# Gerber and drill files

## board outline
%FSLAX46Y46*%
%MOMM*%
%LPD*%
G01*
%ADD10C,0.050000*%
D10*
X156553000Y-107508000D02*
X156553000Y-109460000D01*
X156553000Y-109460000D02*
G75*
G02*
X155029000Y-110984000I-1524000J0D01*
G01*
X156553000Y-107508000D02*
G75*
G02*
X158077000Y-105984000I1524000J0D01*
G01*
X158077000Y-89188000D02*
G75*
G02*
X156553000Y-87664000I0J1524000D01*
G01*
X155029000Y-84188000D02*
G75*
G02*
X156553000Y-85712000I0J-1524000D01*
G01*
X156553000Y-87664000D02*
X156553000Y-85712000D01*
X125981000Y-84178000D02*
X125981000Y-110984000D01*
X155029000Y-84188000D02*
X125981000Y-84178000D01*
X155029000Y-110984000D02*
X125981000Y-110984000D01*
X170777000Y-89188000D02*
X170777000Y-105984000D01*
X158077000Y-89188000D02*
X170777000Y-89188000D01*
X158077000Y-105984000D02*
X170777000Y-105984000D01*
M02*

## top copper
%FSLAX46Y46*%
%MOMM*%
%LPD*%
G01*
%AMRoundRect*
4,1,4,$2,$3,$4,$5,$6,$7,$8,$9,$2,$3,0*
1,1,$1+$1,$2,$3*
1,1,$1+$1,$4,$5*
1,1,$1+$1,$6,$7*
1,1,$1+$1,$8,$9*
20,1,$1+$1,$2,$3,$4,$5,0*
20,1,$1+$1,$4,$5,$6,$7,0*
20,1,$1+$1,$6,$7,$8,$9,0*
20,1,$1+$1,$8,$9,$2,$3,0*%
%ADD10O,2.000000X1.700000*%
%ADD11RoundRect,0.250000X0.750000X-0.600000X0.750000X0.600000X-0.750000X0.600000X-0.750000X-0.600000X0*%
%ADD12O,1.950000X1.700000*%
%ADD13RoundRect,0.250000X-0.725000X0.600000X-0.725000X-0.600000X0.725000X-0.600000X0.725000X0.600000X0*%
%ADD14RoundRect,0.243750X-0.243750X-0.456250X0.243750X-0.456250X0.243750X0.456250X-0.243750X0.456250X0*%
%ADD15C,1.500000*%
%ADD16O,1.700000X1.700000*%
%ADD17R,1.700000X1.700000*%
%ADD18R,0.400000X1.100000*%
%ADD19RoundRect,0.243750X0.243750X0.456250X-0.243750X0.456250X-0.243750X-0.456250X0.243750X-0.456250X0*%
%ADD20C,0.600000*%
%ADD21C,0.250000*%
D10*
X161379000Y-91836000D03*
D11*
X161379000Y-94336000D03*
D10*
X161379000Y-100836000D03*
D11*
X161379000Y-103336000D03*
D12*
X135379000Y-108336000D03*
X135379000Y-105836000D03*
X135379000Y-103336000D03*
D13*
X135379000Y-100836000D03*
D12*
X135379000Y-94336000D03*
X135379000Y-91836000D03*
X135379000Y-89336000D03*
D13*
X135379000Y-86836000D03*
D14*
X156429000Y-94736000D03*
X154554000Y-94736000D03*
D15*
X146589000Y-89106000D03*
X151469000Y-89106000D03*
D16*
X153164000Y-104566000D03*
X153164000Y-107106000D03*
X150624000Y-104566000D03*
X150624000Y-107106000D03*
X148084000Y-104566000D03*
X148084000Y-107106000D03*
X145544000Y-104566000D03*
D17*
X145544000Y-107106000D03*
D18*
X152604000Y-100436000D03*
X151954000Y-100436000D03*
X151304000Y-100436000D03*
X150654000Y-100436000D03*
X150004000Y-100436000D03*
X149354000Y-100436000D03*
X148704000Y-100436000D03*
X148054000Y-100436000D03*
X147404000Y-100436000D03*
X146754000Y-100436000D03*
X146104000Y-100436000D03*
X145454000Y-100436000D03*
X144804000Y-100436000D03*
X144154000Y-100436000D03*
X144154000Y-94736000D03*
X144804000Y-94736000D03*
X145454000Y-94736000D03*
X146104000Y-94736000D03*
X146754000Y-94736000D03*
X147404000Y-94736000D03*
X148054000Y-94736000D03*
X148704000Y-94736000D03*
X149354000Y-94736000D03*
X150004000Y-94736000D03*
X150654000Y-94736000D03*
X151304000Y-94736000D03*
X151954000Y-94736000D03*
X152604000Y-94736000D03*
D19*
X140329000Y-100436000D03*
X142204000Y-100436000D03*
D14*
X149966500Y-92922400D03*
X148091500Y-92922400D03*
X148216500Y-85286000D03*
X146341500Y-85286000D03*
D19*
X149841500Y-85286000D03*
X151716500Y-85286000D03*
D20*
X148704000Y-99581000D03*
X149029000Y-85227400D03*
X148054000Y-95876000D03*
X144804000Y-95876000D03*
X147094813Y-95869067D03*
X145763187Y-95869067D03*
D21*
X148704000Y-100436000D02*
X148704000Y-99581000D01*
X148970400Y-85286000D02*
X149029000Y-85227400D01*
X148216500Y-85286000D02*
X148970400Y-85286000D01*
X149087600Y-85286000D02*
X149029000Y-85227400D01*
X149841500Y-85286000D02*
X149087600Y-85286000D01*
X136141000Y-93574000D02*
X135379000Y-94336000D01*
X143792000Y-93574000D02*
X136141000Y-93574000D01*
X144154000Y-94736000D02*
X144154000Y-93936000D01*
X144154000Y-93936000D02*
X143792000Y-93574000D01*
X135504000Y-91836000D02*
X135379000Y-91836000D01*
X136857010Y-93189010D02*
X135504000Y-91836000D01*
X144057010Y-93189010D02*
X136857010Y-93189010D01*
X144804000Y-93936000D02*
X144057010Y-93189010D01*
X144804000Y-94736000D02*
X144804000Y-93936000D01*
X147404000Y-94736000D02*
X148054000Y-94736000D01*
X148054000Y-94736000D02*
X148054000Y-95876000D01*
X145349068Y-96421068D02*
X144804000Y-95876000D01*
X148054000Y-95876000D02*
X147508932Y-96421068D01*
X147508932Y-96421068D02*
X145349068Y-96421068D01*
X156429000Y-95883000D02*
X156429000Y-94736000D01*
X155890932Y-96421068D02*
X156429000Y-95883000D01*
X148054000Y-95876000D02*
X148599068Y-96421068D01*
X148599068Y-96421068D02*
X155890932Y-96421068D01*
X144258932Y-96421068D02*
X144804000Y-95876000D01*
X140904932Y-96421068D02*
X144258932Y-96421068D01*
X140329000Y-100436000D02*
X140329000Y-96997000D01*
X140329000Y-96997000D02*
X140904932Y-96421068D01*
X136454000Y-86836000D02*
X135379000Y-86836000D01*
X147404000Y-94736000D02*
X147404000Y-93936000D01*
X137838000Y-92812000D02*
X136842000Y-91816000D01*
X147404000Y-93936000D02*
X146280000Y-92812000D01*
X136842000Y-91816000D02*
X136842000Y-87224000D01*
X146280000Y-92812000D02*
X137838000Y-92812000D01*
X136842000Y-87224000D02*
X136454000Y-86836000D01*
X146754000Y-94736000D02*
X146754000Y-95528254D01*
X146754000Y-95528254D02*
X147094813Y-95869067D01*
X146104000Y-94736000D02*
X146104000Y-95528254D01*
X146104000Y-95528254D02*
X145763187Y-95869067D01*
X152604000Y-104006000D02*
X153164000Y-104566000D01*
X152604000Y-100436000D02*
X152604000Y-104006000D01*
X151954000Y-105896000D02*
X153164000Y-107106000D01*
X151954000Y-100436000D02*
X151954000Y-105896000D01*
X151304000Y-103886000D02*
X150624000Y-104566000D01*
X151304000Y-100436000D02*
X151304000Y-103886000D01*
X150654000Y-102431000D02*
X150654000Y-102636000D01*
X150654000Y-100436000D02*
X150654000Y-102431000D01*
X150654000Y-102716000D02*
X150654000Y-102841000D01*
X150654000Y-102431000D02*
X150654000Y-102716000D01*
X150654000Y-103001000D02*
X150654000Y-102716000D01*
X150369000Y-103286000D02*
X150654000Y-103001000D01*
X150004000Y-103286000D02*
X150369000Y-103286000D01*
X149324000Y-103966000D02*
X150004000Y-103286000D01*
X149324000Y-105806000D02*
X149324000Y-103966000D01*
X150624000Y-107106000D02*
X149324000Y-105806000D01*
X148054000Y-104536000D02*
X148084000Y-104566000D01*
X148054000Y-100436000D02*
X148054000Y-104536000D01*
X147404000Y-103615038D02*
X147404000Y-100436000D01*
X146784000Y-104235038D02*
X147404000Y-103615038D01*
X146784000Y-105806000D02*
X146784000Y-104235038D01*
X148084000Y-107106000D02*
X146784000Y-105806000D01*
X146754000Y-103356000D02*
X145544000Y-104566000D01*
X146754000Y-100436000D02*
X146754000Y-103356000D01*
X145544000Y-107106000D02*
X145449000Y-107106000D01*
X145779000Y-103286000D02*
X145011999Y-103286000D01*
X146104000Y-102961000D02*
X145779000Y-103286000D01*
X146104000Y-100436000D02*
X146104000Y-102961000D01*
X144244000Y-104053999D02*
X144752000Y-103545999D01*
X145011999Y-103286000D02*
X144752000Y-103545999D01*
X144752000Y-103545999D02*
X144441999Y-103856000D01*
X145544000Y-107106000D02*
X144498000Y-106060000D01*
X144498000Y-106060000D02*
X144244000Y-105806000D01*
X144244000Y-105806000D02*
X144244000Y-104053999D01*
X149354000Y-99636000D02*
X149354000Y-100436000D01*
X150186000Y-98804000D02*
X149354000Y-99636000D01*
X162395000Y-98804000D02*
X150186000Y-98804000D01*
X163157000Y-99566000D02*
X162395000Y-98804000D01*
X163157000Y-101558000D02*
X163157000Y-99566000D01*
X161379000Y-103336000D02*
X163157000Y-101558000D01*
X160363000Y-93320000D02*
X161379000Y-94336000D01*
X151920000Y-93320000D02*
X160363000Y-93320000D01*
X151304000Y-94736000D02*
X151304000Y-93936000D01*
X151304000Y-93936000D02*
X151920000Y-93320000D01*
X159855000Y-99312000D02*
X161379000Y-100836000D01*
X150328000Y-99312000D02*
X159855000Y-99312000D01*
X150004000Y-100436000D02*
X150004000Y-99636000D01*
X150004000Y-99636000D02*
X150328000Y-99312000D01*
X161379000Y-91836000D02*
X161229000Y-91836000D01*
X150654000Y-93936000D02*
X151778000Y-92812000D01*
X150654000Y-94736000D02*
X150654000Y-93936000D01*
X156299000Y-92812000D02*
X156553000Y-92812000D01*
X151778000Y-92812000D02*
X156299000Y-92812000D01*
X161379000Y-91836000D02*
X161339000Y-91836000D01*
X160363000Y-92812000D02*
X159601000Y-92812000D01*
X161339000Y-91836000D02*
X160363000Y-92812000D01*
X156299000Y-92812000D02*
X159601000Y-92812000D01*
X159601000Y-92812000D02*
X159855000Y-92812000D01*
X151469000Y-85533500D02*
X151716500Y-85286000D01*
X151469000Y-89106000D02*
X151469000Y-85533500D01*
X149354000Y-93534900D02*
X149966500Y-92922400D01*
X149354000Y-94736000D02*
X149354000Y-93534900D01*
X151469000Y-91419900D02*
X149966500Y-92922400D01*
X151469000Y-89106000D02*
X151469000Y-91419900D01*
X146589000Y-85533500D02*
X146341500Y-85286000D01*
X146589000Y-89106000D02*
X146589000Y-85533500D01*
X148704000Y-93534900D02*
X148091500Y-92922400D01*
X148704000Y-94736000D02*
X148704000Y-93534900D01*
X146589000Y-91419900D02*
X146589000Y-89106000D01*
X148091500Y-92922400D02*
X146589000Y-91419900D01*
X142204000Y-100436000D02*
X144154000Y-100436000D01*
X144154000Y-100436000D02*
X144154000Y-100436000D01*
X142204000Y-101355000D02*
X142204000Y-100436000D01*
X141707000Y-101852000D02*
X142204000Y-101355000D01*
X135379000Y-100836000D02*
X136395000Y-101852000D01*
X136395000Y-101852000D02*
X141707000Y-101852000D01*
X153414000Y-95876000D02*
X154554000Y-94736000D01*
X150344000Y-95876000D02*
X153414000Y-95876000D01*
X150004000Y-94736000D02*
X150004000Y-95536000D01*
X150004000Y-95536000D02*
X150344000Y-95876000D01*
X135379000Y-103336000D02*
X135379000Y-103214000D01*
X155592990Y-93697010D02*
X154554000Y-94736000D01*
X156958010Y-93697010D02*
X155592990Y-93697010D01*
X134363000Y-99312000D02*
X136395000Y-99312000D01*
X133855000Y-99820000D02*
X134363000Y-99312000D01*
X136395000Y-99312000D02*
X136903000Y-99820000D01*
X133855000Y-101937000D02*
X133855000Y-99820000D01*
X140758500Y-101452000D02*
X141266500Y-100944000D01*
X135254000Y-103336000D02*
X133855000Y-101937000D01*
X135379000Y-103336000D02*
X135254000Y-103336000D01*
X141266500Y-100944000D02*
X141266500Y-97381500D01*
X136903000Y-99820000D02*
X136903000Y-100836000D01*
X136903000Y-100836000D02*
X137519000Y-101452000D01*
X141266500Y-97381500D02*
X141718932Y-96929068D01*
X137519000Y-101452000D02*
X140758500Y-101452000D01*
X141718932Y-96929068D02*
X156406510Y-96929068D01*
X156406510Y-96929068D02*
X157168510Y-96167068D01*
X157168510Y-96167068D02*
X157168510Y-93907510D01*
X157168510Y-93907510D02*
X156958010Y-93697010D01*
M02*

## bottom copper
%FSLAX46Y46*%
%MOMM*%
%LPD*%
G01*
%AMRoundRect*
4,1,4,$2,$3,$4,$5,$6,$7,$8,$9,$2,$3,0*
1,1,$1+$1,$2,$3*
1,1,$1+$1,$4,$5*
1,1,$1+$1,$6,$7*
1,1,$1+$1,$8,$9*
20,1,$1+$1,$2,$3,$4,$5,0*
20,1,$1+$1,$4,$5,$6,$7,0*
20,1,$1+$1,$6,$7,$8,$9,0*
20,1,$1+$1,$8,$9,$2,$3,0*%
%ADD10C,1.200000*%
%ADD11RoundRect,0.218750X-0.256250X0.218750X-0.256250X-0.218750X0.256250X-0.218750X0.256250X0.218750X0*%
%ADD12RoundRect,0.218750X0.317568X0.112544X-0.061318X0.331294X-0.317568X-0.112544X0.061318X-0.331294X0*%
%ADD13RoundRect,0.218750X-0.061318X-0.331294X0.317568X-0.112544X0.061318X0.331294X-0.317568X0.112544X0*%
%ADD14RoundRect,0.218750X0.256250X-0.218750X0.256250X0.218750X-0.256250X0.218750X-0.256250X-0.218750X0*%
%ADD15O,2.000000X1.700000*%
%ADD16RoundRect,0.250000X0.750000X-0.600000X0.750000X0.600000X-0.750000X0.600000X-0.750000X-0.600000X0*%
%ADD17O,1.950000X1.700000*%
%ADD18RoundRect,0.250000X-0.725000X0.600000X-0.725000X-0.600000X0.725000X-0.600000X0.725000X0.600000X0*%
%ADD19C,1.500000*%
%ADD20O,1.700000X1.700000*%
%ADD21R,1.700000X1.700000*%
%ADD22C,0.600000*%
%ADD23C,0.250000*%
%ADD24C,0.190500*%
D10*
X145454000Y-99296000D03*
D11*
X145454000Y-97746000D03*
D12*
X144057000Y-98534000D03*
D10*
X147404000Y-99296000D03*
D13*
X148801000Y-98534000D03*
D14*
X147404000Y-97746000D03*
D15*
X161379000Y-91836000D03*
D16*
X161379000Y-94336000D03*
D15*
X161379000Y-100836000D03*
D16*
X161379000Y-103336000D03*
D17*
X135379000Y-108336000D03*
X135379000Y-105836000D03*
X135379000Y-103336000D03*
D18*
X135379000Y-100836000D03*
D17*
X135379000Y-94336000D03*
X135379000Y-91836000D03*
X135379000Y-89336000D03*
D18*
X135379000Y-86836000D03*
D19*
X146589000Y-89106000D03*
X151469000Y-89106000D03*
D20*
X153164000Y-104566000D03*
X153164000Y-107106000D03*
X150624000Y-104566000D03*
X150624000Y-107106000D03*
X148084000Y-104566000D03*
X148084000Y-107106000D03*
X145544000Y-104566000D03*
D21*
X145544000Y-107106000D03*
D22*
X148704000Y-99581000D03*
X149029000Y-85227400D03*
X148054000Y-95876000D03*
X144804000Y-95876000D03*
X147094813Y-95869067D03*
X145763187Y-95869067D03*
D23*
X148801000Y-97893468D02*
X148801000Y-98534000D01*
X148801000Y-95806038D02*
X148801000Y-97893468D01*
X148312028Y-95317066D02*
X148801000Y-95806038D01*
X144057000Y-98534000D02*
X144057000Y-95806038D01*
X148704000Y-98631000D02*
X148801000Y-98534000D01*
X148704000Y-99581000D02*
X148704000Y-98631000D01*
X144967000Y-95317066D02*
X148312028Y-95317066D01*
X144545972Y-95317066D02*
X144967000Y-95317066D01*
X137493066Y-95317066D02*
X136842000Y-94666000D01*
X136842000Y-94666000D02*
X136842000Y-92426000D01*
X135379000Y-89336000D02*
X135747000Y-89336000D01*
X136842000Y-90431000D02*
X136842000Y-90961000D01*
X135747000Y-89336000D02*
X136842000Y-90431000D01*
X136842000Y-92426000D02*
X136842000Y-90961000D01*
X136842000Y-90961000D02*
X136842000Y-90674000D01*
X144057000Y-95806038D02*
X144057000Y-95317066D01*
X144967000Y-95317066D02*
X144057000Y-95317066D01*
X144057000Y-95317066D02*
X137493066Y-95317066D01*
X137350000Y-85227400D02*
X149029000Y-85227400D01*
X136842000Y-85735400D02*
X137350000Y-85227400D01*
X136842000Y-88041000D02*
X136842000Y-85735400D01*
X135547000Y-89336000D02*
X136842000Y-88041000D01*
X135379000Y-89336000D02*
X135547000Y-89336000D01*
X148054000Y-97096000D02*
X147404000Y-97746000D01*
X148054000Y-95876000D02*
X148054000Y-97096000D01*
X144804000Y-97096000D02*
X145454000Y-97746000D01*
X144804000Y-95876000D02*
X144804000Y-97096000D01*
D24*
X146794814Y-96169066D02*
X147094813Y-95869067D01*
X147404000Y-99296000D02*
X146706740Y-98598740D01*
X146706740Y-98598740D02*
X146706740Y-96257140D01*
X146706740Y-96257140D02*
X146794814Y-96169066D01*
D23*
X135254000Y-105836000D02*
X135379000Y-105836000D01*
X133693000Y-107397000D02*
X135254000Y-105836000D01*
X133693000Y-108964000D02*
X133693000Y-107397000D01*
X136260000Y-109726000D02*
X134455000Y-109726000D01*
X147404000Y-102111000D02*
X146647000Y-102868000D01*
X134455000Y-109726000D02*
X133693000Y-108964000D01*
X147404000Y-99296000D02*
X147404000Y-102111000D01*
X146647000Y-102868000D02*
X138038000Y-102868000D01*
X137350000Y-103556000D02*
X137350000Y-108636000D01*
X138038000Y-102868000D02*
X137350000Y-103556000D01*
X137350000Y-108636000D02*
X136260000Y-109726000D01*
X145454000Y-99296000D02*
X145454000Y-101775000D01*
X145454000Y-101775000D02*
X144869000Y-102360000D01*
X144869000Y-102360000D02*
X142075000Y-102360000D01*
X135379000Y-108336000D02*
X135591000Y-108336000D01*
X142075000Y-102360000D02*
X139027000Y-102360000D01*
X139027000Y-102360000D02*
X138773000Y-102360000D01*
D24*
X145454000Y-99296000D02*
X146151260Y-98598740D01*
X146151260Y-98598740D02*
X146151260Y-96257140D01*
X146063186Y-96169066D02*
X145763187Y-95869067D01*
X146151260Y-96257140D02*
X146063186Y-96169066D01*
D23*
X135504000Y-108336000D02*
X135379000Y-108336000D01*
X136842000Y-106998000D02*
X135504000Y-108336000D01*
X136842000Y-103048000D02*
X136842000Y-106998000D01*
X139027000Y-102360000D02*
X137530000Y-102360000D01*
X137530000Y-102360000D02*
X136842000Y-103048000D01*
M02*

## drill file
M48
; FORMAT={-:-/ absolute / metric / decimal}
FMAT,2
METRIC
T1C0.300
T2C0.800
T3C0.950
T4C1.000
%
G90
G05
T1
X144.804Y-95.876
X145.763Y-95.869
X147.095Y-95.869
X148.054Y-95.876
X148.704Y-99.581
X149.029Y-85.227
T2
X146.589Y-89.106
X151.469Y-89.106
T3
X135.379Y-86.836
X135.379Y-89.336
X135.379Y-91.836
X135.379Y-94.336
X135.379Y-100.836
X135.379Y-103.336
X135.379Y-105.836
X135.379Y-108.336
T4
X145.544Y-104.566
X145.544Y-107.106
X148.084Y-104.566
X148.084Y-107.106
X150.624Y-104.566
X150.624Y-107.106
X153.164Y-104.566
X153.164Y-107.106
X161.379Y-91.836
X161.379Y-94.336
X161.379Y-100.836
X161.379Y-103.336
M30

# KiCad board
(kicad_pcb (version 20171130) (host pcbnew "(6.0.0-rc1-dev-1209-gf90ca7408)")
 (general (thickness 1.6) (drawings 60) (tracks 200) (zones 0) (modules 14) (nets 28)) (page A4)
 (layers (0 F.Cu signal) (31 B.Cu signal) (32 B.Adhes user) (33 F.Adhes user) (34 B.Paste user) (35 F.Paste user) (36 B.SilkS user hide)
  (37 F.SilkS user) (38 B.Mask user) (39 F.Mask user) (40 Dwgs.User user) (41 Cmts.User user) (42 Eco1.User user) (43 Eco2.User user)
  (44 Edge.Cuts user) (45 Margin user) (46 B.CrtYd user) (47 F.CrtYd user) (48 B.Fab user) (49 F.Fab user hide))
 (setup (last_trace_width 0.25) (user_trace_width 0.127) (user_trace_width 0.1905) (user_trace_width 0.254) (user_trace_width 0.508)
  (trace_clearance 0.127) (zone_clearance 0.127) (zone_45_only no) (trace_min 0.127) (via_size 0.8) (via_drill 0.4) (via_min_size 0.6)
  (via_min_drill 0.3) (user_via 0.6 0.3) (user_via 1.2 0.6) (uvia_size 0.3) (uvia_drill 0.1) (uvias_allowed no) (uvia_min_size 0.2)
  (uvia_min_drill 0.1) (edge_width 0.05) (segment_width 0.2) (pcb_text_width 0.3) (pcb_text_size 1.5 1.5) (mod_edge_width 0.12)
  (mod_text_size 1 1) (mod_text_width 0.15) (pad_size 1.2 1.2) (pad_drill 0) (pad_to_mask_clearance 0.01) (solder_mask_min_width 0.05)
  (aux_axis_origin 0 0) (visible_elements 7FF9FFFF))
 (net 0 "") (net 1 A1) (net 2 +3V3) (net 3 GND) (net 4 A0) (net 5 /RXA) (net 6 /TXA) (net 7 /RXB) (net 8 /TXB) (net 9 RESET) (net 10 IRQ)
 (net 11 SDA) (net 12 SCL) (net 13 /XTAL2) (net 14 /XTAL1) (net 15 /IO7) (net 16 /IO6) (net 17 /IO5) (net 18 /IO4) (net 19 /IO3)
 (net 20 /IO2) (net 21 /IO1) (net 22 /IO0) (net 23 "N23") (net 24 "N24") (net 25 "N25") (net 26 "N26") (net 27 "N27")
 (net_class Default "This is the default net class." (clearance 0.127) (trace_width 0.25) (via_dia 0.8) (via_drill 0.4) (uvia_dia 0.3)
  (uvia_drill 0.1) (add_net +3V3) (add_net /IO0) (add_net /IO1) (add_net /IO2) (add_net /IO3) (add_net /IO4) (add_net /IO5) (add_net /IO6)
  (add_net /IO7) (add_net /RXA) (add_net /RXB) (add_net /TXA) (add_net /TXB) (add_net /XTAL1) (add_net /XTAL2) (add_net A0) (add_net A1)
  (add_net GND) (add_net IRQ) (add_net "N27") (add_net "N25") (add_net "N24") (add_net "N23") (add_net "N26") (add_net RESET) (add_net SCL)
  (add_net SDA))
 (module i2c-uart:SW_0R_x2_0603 (layer B.Cu) (at 145.454 99.296)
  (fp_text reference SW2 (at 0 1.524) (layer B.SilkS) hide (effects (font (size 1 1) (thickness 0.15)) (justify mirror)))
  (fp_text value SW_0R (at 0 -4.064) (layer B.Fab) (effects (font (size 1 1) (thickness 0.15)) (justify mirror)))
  (pad 2 smd circle (at 0 0) (size 1.2 1.2) (layers B.Cu B.Paste B.Mask) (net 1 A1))
  (pad 1 smd roundrect (at 0 -1.55 270) (size 0.875 0.95) (layers B.Cu B.Paste B.Mask) (roundrect_rratio 0.25) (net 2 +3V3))
  (pad 3 smd roundrect (at -1.397 -0.762 150) (size 0.875 0.95) (layers B.Cu B.Paste B.Mask) (roundrect_rratio 0.25) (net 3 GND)))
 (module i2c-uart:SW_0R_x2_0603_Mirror (layer B.Cu) (at 147.404 99.296 180)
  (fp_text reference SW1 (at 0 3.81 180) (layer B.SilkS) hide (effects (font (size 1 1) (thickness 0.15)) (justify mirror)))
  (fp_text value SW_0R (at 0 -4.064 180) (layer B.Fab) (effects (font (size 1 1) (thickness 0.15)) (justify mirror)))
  (pad 2 smd circle (at 0 0 180) (size 1.2 1.2) (layers B.Cu B.Paste B.Mask) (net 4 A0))
  (pad 3 smd roundrect (at -1.397 0.762 30) (size 0.875 0.95) (layers B.Cu B.Paste B.Mask) (roundrect_rratio 0.25) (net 3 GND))
  (pad 1 smd roundrect (at 0 1.55 90) (size 0.875 0.95) (layers B.Cu B.Paste B.Mask) (roundrect_rratio 0.25) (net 2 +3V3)))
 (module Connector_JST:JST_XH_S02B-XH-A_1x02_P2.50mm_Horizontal (layer F.Cu) (at 161.379 94.336 90)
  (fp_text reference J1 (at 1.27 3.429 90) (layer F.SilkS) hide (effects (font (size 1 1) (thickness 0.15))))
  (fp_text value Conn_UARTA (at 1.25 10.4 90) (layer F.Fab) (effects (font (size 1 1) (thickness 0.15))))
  (pad 2 thru_hole oval (at 2.5 0 90) (size 1.7 2) (drill 1) (layers *.Cu *.Mask) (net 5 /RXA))
  (pad 1 thru_hole roundrect (at 0 0 90) (size 1.7 2) (drill 1) (layers *.Cu *.Mask) (roundrect_rratio 0.147059) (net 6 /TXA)))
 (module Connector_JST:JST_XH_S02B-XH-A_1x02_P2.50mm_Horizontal (layer F.Cu) (at 161.379 103.336 90)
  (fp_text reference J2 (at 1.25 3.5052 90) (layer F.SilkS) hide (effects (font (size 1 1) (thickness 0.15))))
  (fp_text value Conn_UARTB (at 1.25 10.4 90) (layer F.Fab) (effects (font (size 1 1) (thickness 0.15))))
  (pad 2 thru_hole oval (at 2.5 0 90) (size 1.7 2) (drill 1) (layers *.Cu *.Mask) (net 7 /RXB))
  (pad 1 thru_hole roundrect (at 0 0 90) (size 1.7 2) (drill 1) (layers *.Cu *.Mask) (roundrect_rratio 0.147059) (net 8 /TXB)))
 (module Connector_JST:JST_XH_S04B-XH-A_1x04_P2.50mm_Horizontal (layer F.Cu) (at 135.379 100.836 270)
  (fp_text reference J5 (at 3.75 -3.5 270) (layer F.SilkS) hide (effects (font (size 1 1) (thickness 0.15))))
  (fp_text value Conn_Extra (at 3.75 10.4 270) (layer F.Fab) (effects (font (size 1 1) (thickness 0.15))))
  (pad 4 thru_hole oval (at 7.5 0 270) (size 1.7 1.95) (drill 0.95) (layers *.Cu *.Mask) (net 1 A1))
  (pad 3 thru_hole oval (at 5 0 270) (size 1.7 1.95) (drill 0.95) (layers *.Cu *.Mask) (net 4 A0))
  (pad 2 thru_hole oval (at 2.5 0 270) (size 1.7 1.95) (drill 0.95) (layers *.Cu *.Mask) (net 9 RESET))
  (pad 1 thru_hole roundrect (at 0 0 270) (size 1.7 1.95) (drill 0.95) (layers *.Cu *.Mask) (roundrect_rratio 0.147059) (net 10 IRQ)))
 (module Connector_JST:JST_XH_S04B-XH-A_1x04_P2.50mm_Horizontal (layer F.Cu) (at 135.379 86.836 270)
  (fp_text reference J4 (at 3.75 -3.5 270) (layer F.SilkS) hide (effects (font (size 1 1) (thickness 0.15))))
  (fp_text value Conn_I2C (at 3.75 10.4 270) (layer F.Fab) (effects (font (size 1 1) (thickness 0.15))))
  (pad 4 thru_hole oval (at 7.5 0 270) (size 1.7 1.95) (drill 0.95) (layers *.Cu *.Mask) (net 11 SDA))
  (pad 3 thru_hole oval (at 5 0 270) (size 1.7 1.95) (drill 0.95) (layers *.Cu *.Mask) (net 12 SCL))
  (pad 2 thru_hole oval (at 2.5 0 270) (size 1.7 1.95) (drill 0.95) (layers *.Cu *.Mask) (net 3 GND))
  (pad 1 thru_hole roundrect (at 0 0 270) (size 1.7 1.95) (drill 0.95) (layers *.Cu *.Mask) (roundrect_rratio 0.147059) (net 2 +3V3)))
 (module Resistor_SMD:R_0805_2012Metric (layer F.Cu) (at 155.4915 94.736)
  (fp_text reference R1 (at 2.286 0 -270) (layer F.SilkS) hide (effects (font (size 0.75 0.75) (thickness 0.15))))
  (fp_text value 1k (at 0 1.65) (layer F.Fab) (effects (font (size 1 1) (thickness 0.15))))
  (pad 2 smd roundrect (at 0.9375 0) (size 0.975 1.4) (layers F.Cu F.Paste F.Mask) (roundrect_rratio 0.25) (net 2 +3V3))
  (pad 1 smd roundrect (at -0.9375 0) (size 0.975 1.4) (layers F.Cu F.Paste F.Mask) (roundrect_rratio 0.25) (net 9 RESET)))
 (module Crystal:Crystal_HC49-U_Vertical (layer F.Cu) (at 151.469 89.106 180)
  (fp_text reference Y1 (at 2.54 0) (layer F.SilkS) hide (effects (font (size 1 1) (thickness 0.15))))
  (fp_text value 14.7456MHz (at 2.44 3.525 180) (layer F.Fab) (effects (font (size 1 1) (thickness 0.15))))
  (pad 2 thru_hole circle (at 4.88 0 180) (size 1.5 1.5) (drill 0.8) (layers *.Cu *.Mask) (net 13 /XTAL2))
  (pad 1 thru_hole circle (at 0 0 180) (size 1.5 1.5) (drill 0.8) (layers *.Cu *.Mask) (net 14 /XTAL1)))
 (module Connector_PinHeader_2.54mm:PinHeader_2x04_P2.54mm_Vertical (layer F.Cu) (at 145.544 107.106 90)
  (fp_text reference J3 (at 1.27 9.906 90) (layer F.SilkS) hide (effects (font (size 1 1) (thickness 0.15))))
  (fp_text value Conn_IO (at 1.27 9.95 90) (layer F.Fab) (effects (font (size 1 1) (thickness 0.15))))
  (pad 8 thru_hole oval (at 2.54 7.62 90) (size 1.7 1.7) (drill 1) (layers *.Cu *.Mask) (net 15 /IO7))
  (pad 7 thru_hole oval (at 0 7.62 90) (size 1.7 1.7) (drill 1) (layers *.Cu *.Mask) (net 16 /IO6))
  (pad 6 thru_hole oval (at 2.54 5.08 90) (size 1.7 1.7) (drill 1) (layers *.Cu *.Mask) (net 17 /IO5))
  (pad 5 thru_hole oval (at 0 5.08 90) (size 1.7 1.7) (drill 1) (layers *.Cu *.Mask) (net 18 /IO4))
  (pad 4 thru_hole oval (at 2.54 2.54 90) (size 1.7 1.7) (drill 1) (layers *.Cu *.Mask) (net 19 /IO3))
  (pad 3 thru_hole oval (at 0 2.54 90) (size 1.7 1.7) (drill 1) (layers *.Cu *.Mask) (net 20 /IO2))
  (pad 2 thru_hole oval (at 2.54 0 90) (size 1.7 1.7) (drill 1) (layers *.Cu *.Mask) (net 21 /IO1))
  (pad 1 thru_hole rect (at 0 0 90) (size 1.7 1.7) (drill 1) (layers *.Cu *.Mask) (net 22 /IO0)))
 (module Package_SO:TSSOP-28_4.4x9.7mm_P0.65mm (layer F.Cu) (at 148.379 97.586 270)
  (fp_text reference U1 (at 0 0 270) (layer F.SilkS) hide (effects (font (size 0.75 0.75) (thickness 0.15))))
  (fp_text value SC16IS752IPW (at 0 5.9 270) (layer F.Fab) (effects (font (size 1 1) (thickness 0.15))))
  (pad 28 smd rect (at 2.85 -4.225 270) (size 1.1 0.4) (layers F.Cu F.Paste F.Mask) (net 15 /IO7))
  (pad 27 smd rect (at 2.85 -3.575 270) (size 1.1 0.4) (layers F.Cu F.Paste F.Mask) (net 16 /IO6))
  (pad 26 smd rect (at 2.85 -2.925 270) (size 1.1 0.4) (layers F.Cu F.Paste F.Mask) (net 17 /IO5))
  (pad 25 smd rect (at 2.85 -2.275 270) (size 1.1 0.4) (layers F.Cu F.Paste F.Mask) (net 18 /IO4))
  (pad 24 smd rect (at 2.85 -1.625 270) (size 1.1 0.4) (layers F.Cu F.Paste F.Mask) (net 7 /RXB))
  (pad 23 smd rect (at 2.85 -0.975 270) (size 1.1 0.4) (layers F.Cu F.Paste F.Mask) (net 8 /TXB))
  (pad 22 smd rect (at 2.85 -0.325 270) (size 1.1 0.4) (layers F.Cu F.Paste F.Mask) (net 3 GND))
  (pad 21 smd rect (at 2.85 0.325 270) (size 1.1 0.4) (layers F.Cu F.Paste F.Mask) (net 19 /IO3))
  (pad 20 smd rect (at 2.85 0.975 270) (size 1.1 0.4) (layers F.Cu F.Paste F.Mask) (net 20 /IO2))
  (pad 19 smd rect (at 2.85 1.625 270) (size 1.1 0.4) (layers F.Cu F.Paste F.Mask) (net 21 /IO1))
  (pad 18 smd rect (at 2.85 2.275 270) (size 1.1 0.4) (layers F.Cu F.Paste F.Mask) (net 22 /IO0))
  (pad 17 smd rect (at 2.85 2.925 270) (size 1.1 0.4) (layers F.Cu F.Paste F.Mask) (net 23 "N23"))
  (pad 16 smd rect (at 2.85 3.575 270) (size 1.1 0.4) (layers F.Cu F.Paste F.Mask) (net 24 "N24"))
  (pad 15 smd rect (at 2.85 4.225 270) (size 1.1 0.4) (layers F.Cu F.Paste F.Mask) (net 10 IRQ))
  (pad 14 smd rect (at -2.85 4.225 270) (size 1.1 0.4) (layers F.Cu F.Paste F.Mask) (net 11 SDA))
  (pad 13 smd rect (at -2.85 3.575 270) (size 1.1 0.4) (layers F.Cu F.Paste F.Mask) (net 12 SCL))
  (pad 12 smd rect (at -2.85 2.925 270) (size 1.1 0.4) (layers F.Cu F.Paste F.Mask) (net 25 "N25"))
  (pad 11 smd rect (at -2.85 2.275 270) (size 1.1 0.4) (layers F.Cu F.Paste F.Mask) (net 1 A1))
  (pad 10 smd rect (at -2.85 1.625 270) (size 1.1 0.4) (layers F.Cu F.Paste F.Mask) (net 4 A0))
  (pad 9 smd rect (at -2.85 0.975 270) (size 1.1 0.4) (layers F.Cu F.Paste F.Mask) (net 2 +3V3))
  (pad 8 smd rect (at -2.85 0.325 270) (size 1.1 0.4) (layers F.Cu F.Paste F.Mask) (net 2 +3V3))
  (pad 7 smd rect (at -2.85 -0.325 270) (size 1.1 0.4) (layers F.Cu F.Paste F.Mask) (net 13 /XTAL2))
  (pad 6 smd rect (at -2.85 -0.975 270) (size 1.1 0.4) (layers F.Cu F.Paste F.Mask) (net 14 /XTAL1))
  (pad 5 smd rect (at -2.85 -1.625 270) (size 1.1 0.4) (layers F.Cu F.Paste F.Mask) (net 9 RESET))
  (pad 4 smd rect (at -2.85 -2.275 270) (size 1.1 0.4) (layers F.Cu F.Paste F.Mask) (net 5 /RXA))
  (pad 3 smd rect (at -2.85 -2.925 270) (size 1.1 0.4) (layers F.Cu F.Paste F.Mask) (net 6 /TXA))
  (pad 2 smd rect (at -2.85 -3.575 270) (size 1.1 0.4) (layers F.Cu F.Paste F.Mask) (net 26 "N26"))
  (pad 1 smd rect (at -2.85 -4.225 270) (size 1.1 0.4) (layers F.Cu F.Paste F.Mask) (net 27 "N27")))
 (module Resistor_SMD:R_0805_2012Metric (layer F.Cu) (at 141.2665 100.436 180)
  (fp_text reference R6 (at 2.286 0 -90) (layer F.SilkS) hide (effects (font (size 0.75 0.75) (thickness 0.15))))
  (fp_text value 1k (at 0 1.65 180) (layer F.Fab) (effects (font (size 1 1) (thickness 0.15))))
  (pad 2 smd roundrect (at 0.9375 0 180) (size 0.975 1.4) (layers F.Cu F.Paste F.Mask) (roundrect_rratio 0.25) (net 2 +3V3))
  (pad 1 smd roundrect (at -0.9375 0 180) (size 0.975 1.4) (layers F.Cu F.Paste F.Mask) (roundrect_rratio 0.25) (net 10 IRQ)))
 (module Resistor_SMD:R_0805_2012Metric (layer F.Cu) (at 149.029 92.9224)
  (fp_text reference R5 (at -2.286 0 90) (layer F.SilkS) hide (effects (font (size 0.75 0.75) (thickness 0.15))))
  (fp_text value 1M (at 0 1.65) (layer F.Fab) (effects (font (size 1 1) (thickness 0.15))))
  (pad 2 smd roundrect (at 0.9375 0) (size 0.975 1.4) (layers F.Cu F.Paste F.Mask) (roundrect_rratio 0.25) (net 14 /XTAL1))
  (pad 1 smd roundrect (at -0.9375 0) (size 0.975 1.4) (layers F.Cu F.Paste F.Mask) (roundrect_rratio 0.25) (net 13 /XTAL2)))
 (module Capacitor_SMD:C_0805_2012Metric (layer F.Cu) (at 147.279 85.286)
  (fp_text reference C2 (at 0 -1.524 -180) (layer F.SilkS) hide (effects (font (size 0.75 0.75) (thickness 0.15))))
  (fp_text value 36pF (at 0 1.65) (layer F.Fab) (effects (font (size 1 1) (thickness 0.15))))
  (pad 2 smd roundrect (at 0.9375 0) (size 0.975 1.4) (layers F.Cu F.Paste F.Mask) (roundrect_rratio 0.25) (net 3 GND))
  (pad 1 smd roundrect (at -0.9375 0) (size 0.975 1.4) (layers F.Cu F.Paste F.Mask) (roundrect_rratio 0.25) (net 13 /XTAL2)))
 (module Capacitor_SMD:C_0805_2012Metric (layer F.Cu) (at 150.779 85.286 180)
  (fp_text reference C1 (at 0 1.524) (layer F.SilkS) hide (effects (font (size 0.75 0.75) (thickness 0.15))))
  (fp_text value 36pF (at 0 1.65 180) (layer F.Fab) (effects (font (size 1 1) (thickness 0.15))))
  (pad 2 smd roundrect (at 0.9375 0 180) (size 0.975 1.4) (layers F.Cu F.Paste F.Mask) (roundrect_rratio 0.25) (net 3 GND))
  (pad 1 smd roundrect (at -0.9375 0 180) (size 0.975 1.4) (layers F.Cu F.Paste F.Mask) (roundrect_rratio 0.25) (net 14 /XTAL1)))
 (gr_line (start 156.553 107.508) (end 156.553 109.46) (layer Edge.Cuts) (width 0.05))
 (gr_arc (start 155.029 109.46) (end 155.029 110.984) (angle -90) (layer Edge.Cuts) (width 0.05))
 (gr_arc (start 158.077 107.508) (end 158.077 105.984) (angle -90) (layer Edge.Cuts) (width 0.05))
 (gr_arc (start 158.077 87.664) (end 156.553 87.664) (angle -90) (layer Edge.Cuts) (width 0.05))
 (gr_arc (start 155.029 85.712) (end 156.553 85.712) (angle -90) (layer Edge.Cuts) (width 0.05))
 (gr_line (start 156.553 87.664) (end 156.553 85.712) (layer Edge.Cuts) (width 0.05))
 (gr_line (start 125.981 84.178) (end 125.981 110.984) (layer Edge.Cuts) (width 0.05))
 (gr_line (start 155.029 84.188) (end 125.981 84.178) (layer Edge.Cuts) (width 0.05))
 (gr_line (start 155.029 110.984) (end 125.981 110.984) (layer Edge.Cuts) (width 0.05))
 (gr_line (start 170.777 89.188) (end 170.777 105.984) (layer Edge.Cuts) (width 0.05))
 (gr_line (start 158.077 89.188) (end 170.777 89.188) (layer Edge.Cuts) (width 0.05))
 (gr_line (start 158.077 105.984) (end 170.777 105.984) (layer Edge.Cuts) (width 0.05))
 (segment (start 148.801 97.893468) (end 148.801 98.534) (width 0.25) (layer B.Cu) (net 3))
 (segment (start 148.801 95.806038) (end 148.801 97.893468) (width 0.25) (layer B.Cu) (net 3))
 (segment (start 148.312028 95.317066) (end 148.801 95.806038) (width 0.25) (layer B.Cu) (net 3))
 (segment (start 144.057 98.534) (end 144.057 95.806038) (width 0.25) (layer B.Cu) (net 3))
 (via (at 148.704 99.581) (size 0.6) (drill 0.3) (layers F.Cu B.Cu) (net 3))
 (segment (start 148.704 100.436) (end 148.704 99.581) (width 0.25) (layer F.Cu) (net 3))
 (segment (start 148.704 98.631) (end 148.801 98.534) (width 0.25) (layer B.Cu) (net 3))
 (segment (start 148.704 99.581) (end 148.704 98.631) (width 0.25) (layer B.Cu) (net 3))
 (segment (start 144.967 95.317066) (end 148.312028 95.317066) (width 0.25) (layer B.Cu) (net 3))
 (segment (start 144.545972 95.317066) (end 144.967 95.317066) (width 0.25) (layer B.Cu) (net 3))
 (segment (start 137.493066 95.317066) (end 136.842 94.666) (width 0.25) (layer B.Cu) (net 3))
 (segment (start 136.842 94.666) (end 136.842 92.426) (width 0.25) (layer B.Cu) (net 3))
 (segment (start 135.379 89.336) (end 135.747 89.336) (width 0.25) (layer B.Cu) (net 3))
 (segment (start 136.842 90.431) (end 136.842 90.961) (width 0.25) (layer B.Cu) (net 3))
 (segment (start 135.747 89.336) (end 136.842 90.431) (width 0.25) (layer B.Cu) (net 3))
 (segment (start 136.842 92.426) (end 136.842 90.961) (width 0.25) (layer B.Cu) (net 3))
 (segment (start 136.842 90.961) (end 136.842 90.674) (width 0.25) (layer B.Cu) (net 3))
 (segment (start 144.057 95.806038) (end 144.057 95.317066) (width 0.25) (layer B.Cu) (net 3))
 (segment (start 144.967 95.317066) (end 144.057 95.317066) (width 0.25) (layer B.Cu) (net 3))
 (segment (start 144.057 95.317066) (end 137.493066 95.317066) (width 0.25) (layer B.Cu) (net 3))
 (via (at 149.029 85.2274) (size 0.6) (drill 0.3) (layers F.Cu B.Cu) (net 3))
 (segment (start 148.9704 85.286) (end 149.029 85.2274) (width 0.25) (layer F.Cu) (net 3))
 (segment (start 148.2165 85.286) (end 148.9704 85.286) (width 0.25) (layer F.Cu) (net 3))
 (segment (start 149.0876 85.286) (end 149.029 85.2274) (width 0.25) (layer F.Cu) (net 3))
 (segment (start 149.8415 85.286) (end 149.0876 85.286) (width 0.25) (layer F.Cu) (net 3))
 (segment (start 137.35 85.2274) (end 149.029 85.2274) (width 0.25) (layer B.Cu) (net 3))
 (segment (start 136.842 85.7354) (end 137.35 85.2274) (width 0.25) (layer B.Cu) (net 3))
 (segment (start 136.842 88.041) (end 136.842 85.7354) (width 0.25) (layer B.Cu) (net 3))
 (segment (start 135.547 89.336) (end 136.842 88.041) (width 0.25) (layer B.Cu) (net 3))
 (segment (start 135.379 89.336) (end 135.547 89.336) (width 0.25) (layer B.Cu) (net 3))
 (segment (start 136.141 93.574) (end 135.379 94.336) (width 0.25) (layer F.Cu) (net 11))
 (segment (start 143.792 93.574) (end 136.141 93.574) (width 0.25) (layer F.Cu) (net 11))
 (segment (start 144.154 94.736) (end 144.154 93.936) (width 0.25) (layer F.Cu) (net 11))
 (segment (start 144.154 93.936) (end 143.792 93.574) (width 0.25) (layer F.Cu) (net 11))
 (segment (start 135.504 91.836) (end 135.379 91.836) (width 0.25) (layer F.Cu) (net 12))
 (segment (start 136.85701 93.18901) (end 135.504 91.836) (width 0.25) (layer F.Cu) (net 12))
 (segment (start 144.05701 93.18901) (end 136.85701 93.18901) (width 0.25) (layer F.Cu) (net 12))
 (segment (start 144.804 93.936) (end 144.05701 93.18901) (width 0.25) (layer F.Cu) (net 12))
 (segment (start 144.804 94.736) (end 144.804 93.936) (width 0.25) (layer F.Cu) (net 12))
 (segment (start 147.404 94.736) (end 148.054 94.736) (width 0.25) (layer F.Cu) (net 2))
 (via (at 148.054 95.876) (size 0.6) (drill 0.3) (layers F.Cu B.Cu) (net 2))
 (segment (start 148.054 94.736) (end 148.054 95.876) (width 0.25) (layer F.Cu) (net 2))
 (segment (start 148.054 97.096) (end 147.404 97.746) (width 0.25) (layer B.Cu) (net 2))
 (segment (start 148.054 95.876) (end 148.054 97.096) (width 0.25) (layer B.Cu) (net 2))
 (via (at 144.804 95.876) (size 0.6) (drill 0.3) (layers F.Cu B.Cu) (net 2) (status 1000000))
 (segment (start 145.349068 96.421068) (end 144.804 95.876) (width 0.25) (layer F.Cu) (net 2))
 (segment (start 148.054 95.876) (end 147.508932 96.421068) (width 0.25) (layer F.Cu) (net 2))
 (segment (start 147.508932 96.421068) (end 145.349068 96.421068) (width 0.25) (layer F.Cu) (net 2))
 (segment (start 144.804 97.096) (end 145.454 97.746) (width 0.25) (layer B.Cu) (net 2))
 (segment (start 144.804 95.876) (end 144.804 97.096) (width 0.25) (layer B.Cu) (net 2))
 (segment (start 156.429 95.883) (end 156.429 94.736) (width 0.25) (layer F.Cu) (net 2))
 (segment (start 155.890932 96.421068) (end 156.429 95.883) (width 0.25) (layer F.Cu) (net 2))
 (segment (start 148.054 95.876) (end 148.599068 96.421068) (width 0.25) (layer F.Cu) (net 2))
 (segment (start 148.599068 96.421068) (end 155.890932 96.421068) (width 0.25) (layer F.Cu) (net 2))
 (segment (start 144.258932 96.421068) (end 144.804 95.876) (width 0.25) (layer F.Cu) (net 2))
 (segment (start 140.904932 96.421068) (end 144.258932 96.421068) (width 0.25) (layer F.Cu) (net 2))
 (segment (start 140.329 100.436) (end 140.329 96.997) (width 0.25) (layer F.Cu) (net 2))
 (segment (start 140.329 96.997) (end 140.904932 96.421068) (width 0.25) (layer F.Cu) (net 2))
 (segment (start 136.454 86.836) (end 135.379 86.836) (width 0.25) (layer F.Cu) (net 2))
 (segment (start 147.404 94.736) (end 147.404 93.936) (width 0.25) (layer F.Cu) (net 2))
 (segment (start 137.838 92.812) (end 136.842 91.816) (width 0.25) (layer F.Cu) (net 2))
 (segment (start 147.404 93.936) (end 146.28 92.812) (width 0.25) (layer F.Cu) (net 2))
 (segment (start 136.842 91.816) (end 136.842 87.224) (width 0.25) (layer F.Cu) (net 2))
 (segment (start 146.28 92.812) (end 137.838 92.812) (width 0.25) (layer F.Cu) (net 2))
 (segment (start 136.842 87.224) (end 136.454 86.836) (width 0.25) (layer F.Cu) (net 2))
 (via (at 147.094813 95.869067) (size 0.6) (drill 0.3) (layers F.Cu B.Cu) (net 4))
 (segment (start 146.754 94.736) (end 146.754 95.528254) (width 0.25) (layer F.Cu) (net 4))
 (segment (start 146.754 95.528254) (end 147.094813 95.869067) (width 0.25) (layer F.Cu) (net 4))
 (segment (start 146.794814 96.169066) (end 147.094813 95.869067) (width 0.1905) (layer B.Cu) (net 4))
 (segment (start 147.404 99.296) (end 146.70674 98.59874) (width 0.1905) (layer B.Cu) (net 4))
 (segment (start 146.70674 98.59874) (end 146.70674 96.25714) (width 0.1905) (layer B.Cu) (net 4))
 (segment (start 146.70674 96.25714) (end 146.794814 96.169066) (width 0.1905) (layer B.Cu) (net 4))
 (segment (start 135.254 105.836) (end 135.379 105.836) (width 0.25) (layer B.Cu) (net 4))
 (segment (start 133.693 107.397) (end 135.254 105.836) (width 0.25) (layer B.Cu) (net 4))
 (segment (start 133.693 108.964) (end 133.693 107.397) (width 0.25) (layer B.Cu) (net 4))
 (segment (start 136.26 109.726) (end 134.455 109.726) (width 0.25) (layer B.Cu) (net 4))
 (segment (start 147.404 102.111) (end 146.647 102.868) (width 0.25) (layer B.Cu) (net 4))
 (segment (start 134.455 109.726) (end 133.693 108.964) (width 0.25) (layer B.Cu) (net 4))
 (segment (start 147.404 99.296) (end 147.404 102.111) (width 0.25) (layer B.Cu) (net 4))
 (segment (start 146.647 102.868) (end 138.038 102.868) (width 0.25) (layer B.Cu) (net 4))
 (segment (start 137.35 103.556) (end 137.35 108.636) (width 0.25) (layer B.Cu) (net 4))
 (segment (start 138.038 102.868) (end 137.35 103.556) (width 0.25) (layer B.Cu) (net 4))
 (segment (start 137.35 108.636) (end 136.26 109.726) (width 0.25) (layer B.Cu) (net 4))
 (via (at 145.763187 95.869067) (size 0.6) (drill 0.3) (layers F.Cu B.Cu) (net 1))
 (segment (start 146.104 94.736) (end 146.104 95.528254) (width 0.25) (layer F.Cu) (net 1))
 (segment (start 146.104 95.528254) (end 145.763187 95.869067) (width 0.25) (layer F.Cu) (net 1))
 (segment (start 145.454 99.296) (end 145.454 101.775) (width 0.25) (layer B.Cu) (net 1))
 (segment (start 145.454 101.775) (end 144.869 102.36) (width 0.25) (layer B.Cu) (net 1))
 (segment (start 144.869 102.36) (end 142.075 102.36) (width 0.25) (layer B.Cu) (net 1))
 (segment (start 135.379 108.336) (end 135.591 108.336) (width 0.25) (layer B.Cu) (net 1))
 (segment (start 142.075 102.36) (end 139.027 102.36) (width 0.25) (layer B.Cu) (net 1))
 (segment (start 139.027 102.36) (end 138.773 102.36) (width 0.25) (layer B.Cu) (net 1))
 (segment (start 145.454 99.296) (end 146.15126 98.59874) (width 0.1905) (layer B.Cu) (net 1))
 (segment (start 146.15126 98.59874) (end 146.15126 96.25714) (width 0.1905) (layer B.Cu) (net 1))
 (segment (start 146.063186 96.169066) (end 145.763187 95.869067) (width 0.1905) (layer B.Cu) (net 1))
 (segment (start 146.15126 96.25714) (end 146.063186 96.169066) (width 0.1905) (layer B.Cu) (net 1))
 (segment (start 135.504 108.336) (end 135.379 108.336) (width 0.25) (layer B.Cu) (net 1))
 (segment (start 136.842 106.998) (end 135.504 108.336) (width 0.25) (layer B.Cu) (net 1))
 (segment (start 136.842 103.048) (end 136.842 106.998) (width 0.25) (layer B.Cu) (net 1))
 (segment (start 139.027 102.36) (end 137.53 102.36) (width 0.25) (layer B.Cu) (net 1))
 (segment (start 137.53 102.36) (end 136.842 103.048) (width 0.25) (layer B.Cu) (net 1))
 (segment (start 152.604 104.006) (end 153.164 104.566) (width 0.25) (layer F.Cu) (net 15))
 (segment (start 152.604 100.436) (end 152.604 104.006) (width 0.25) (layer F.Cu) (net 15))
 (segment (start 151.954 105.896) (end 153.164 107.106) (width 0.25) (layer F.Cu) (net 16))
 (segment (start 151.954 100.436) (end 151.954 105.896) (width 0.25) (layer F.Cu) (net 16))
 (segment (start 151.304 103.886) (end 150.624 104.566) (width 0.25) (layer F.Cu) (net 17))
 (segment (start 151.304 100.436) (end 151.304 103.886) (width 0.25) (layer F.Cu) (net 17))
 (segment (start 150.654 102.431) (end 150.654 102.636) (width 0.25) (layer F.Cu) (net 18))
 (segment (start 150.654 100.436) (end 150.654 102.431) (width 0.25) (layer F.Cu) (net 18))
 (segment (start 150.654 102.716) (end 150.654 102.841) (width 0.25) (layer F.Cu) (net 18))
 (segment (start 150.654 102.431) (end 150.654 102.716) (width 0.25) (layer F.Cu) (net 18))
 (segment (start 150.654 103.001) (end 150.654 102.716) (width 0.25) (layer F.Cu) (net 18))
 (segment (start 150.369 103.286) (end 150.654 103.001) (width 0.25) (layer F.Cu) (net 18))
 (segment (start 150.004 103.286) (end 150.369 103.286) (width 0.25) (layer F.Cu) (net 18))
 (segment (start 149.324 103.966) (end 150.004 103.286) (width 0.25) (layer F.Cu) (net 18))
 (segment (start 149.324 105.806) (end 149.324 103.966) (width 0.25) (layer F.Cu) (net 18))
 (segment (start 150.624 107.106) (end 149.324 105.806) (width 0.25) (layer F.Cu) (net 18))
 (segment (start 148.054 104.536) (end 148.084 104.566) (width 0.25) (layer F.Cu) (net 19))
 (segment (start 148.054 100.436) (end 148.054 104.536) (width 0.25) (layer F.Cu) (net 19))
 (segment (start 147.404 103.615038) (end 147.404 100.436) (width 0.25) (layer F.Cu) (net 20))
 (segment (start 146.784 104.235038) (end 147.404 103.615038) (width 0.25) (layer F.Cu) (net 20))
 (segment (start 146.784 105.806) (end 146.784 104.235038) (width 0.25) (layer F.Cu) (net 20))
 (segment (start 148.084 107.106) (end 146.784 105.806) (width 0.25) (layer F.Cu) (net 20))
 (segment (start 146.754 103.356) (end 145.544 104.566) (width 0.25) (layer F.Cu) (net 21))
 (segment (start 146.754 100.436) (end 146.754 103.356) (width 0.25) (layer F.Cu) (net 21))
 (segment (start 145.544 107.106) (end 145.449 107.106) (width 0.25) (layer F.Cu) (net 22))
 (segment (start 145.779 103.286) (end 145.011999 103.286) (width 0.25) (layer F.Cu) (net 22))
 (segment (start 146.104 102.961) (end 145.779 103.286) (width 0.25) (layer F.Cu) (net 22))
 (segment (start 146.104 100.436) (end 146.104 102.961) (width 0.25) (layer F.Cu) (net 22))
 (segment (start 144.244 104.053999) (end 144.752 103.545999) (width 0.25) (layer F.Cu) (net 22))
 (segment (start 145.011999 103.286) (end 144.752 103.545999) (width 0.25) (layer F.Cu) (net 22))
 (segment (start 144.752 103.545999) (end 144.441999 103.856) (width 0.25) (layer F.Cu) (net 22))
 (segment (start 145.544 107.106) (end 144.498 106.06) (width 0.25) (layer F.Cu) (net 22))
 (segment (start 144.498 106.06) (end 144.244 105.806) (width 0.25) (layer F.Cu) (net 22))
 (segment (start 144.244 105.806) (end 144.244 104.053999) (width 0.25) (layer F.Cu) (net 22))
 (segment (start 149.354 99.636) (end 149.354 100.436) (width 0.25) (layer F.Cu) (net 8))
 (segment (start 150.186 98.804) (end 149.354 99.636) (width 0.25) (layer F.Cu) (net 8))
 (segment (start 162.395 98.804) (end 150.186 98.804) (width 0.25) (layer F.Cu) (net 8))
 (segment (start 163.157 99.566) (end 162.395 98.804) (width 0.25) (layer F.Cu) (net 8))
 (segment (start 163.157 101.558) (end 163.157 99.566) (width 0.25) (layer F.Cu) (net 8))
 (segment (start 161.379 103.336) (end 163.157 101.558) (width 0.25) (layer F.Cu) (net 8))
 (segment (start 160.363 93.32) (end 161.379 94.336) (width 0.25) (layer F.Cu) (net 6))
 (segment (start 151.92 93.32) (end 160.363 93.32) (width 0.25) (layer F.Cu) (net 6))
 (segment (start 151.304 94.736) (end 151.304 93.936) (width 0.25) (layer F.Cu) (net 6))
 (segment (start 151.304 93.936) (end 151.92 93.32) (width 0.25) (layer F.Cu) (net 6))
 (segment (start 159.855 99.312) (end 161.379 100.836) (width 0.25) (layer F.Cu) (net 7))
 (segment (start 150.328 99.312) (end 159.855 99.312) (width 0.25) (layer F.Cu) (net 7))
 (segment (start 150.004 100.436) (end 150.004 99.636) (width 0.25) (layer F.Cu) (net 7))
 (segment (start 150.004 99.636) (end 150.328 99.312) (width 0.25) (layer F.Cu) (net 7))
 (segment (start 161.379 91.836) (end 161.229 91.836) (width 0.25) (layer F.Cu) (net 5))
 (segment (start 150.654 93.936) (end 151.778 92.812) (width 0.25) (layer F.Cu) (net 5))
 (segment (start 150.654 94.736) (end 150.654 93.936) (width 0.25) (layer F.Cu) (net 5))
 (segment (start 156.299 92.812) (end 156.553 92.812) (width 0.25) (layer F.Cu) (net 5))
 (segment (start 151.778 92.812) (end 156.299 92.812) (width 0.25) (layer F.Cu) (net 5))
 (segment (start 161.379 91.836) (end 161.339 91.836) (width 0.25) (layer F.Cu) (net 5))
 (segment (start 160.363 92.812) (end 159.601 92.812) (width 0.25) (layer F.Cu) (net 5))
 (segment (start 161.339 91.836) (end 160.363 92.812) (width 0.25) (layer F.Cu) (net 5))
 (segment (start 156.299 92.812) (end 159.601 92.812) (width 0.25) (layer F.Cu) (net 5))
 (segment (start 159.601 92.812) (end 159.855 92.812) (width 0.25) (layer F.Cu) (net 5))
 (segment (start 151.469 85.5335) (end 151.7165 85.286) (width 0.25) (layer F.Cu) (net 14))
 (segment (start 151.469 89.106) (end 151.469 85.5335) (width 0.25) (layer F.Cu) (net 14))
 (segment (start 149.354 93.5349) (end 149.9665 92.9224) (width 0.25) (layer F.Cu) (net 14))
 (segment (start 149.354 94.736) (end 149.354 93.5349) (width 0.25) (layer F.Cu) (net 14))
 (segment (start 151.469 91.4199) (end 149.9665 92.9224) (width 0.25) (layer F.Cu) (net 14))
 (segment (start 151.469 89.106) (end 151.469 91.4199) (width 0.25) (layer F.Cu) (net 14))
 (segment (start 146.589 85.5335) (end 146.3415 85.286) (width 0.25) (layer F.Cu) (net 13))
 (segment (start 146.589 89.106) (end 146.589 85.5335) (width 0.25) (layer F.Cu) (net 13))
 (segment (start 148.704 93.5349) (end 148.0915 92.9224) (width 0.25) (layer F.Cu) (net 13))
 (segment (start 148.704 94.736) (end 148.704 93.5349) (width 0.25) (layer F.Cu) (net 13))
 (segment (start 146.589 91.4199) (end 146.589 89.106) (width 0.25) (layer F.Cu) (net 13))
 (segment (start 148.0915 92.9224) (end 146.589 91.4199) (width 0.25) (layer F.Cu) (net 13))
 (segment (start 142.204 100.436) (end 144.154 100.436) (width 0.25) (layer F.Cu) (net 10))
 (segment (start 144.154 100.436) (end 144.154 100.436) (width 0.25) (layer F.Cu) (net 10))
 (segment (start 142.204 101.355) (end 142.204 100.436) (width 0.25) (layer F.Cu) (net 10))
 (segment (start 141.707 101.852) (end 142.204 101.355) (width 0.25) (layer F.Cu) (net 10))
 (segment (start 135.379 100.836) (end 136.395 101.852) (width 0.25) (layer F.Cu) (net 10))
 (segment (start 136.395 101.852) (end 141.707 101.852) (width 0.25) (layer F.Cu) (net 10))
 (segment (start 153.414 95.876) (end 154.554 94.736) (width 0.25) (layer F.Cu) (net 9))
 (segment (start 150.344 95.876) (end 153.414 95.876) (width 0.25) (layer F.Cu) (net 9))
 (segment (start 150.004 94.736) (end 150.004 95.536) (width 0.25) (layer F.Cu) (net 9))
 (segment (start 150.004 95.536) (end 150.344 95.876) (width 0.25) (layer F.Cu) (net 9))
 (segment (start 135.379 103.336) (end 135.379 103.214) (width 0.25) (layer F.Cu) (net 9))
 (segment (start 155.59299 93.69701) (end 154.554 94.736) (width 0.25) (layer F.Cu) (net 9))
 (segment (start 156.95801 93.69701) (end 155.59299 93.69701) (width 0.25) (layer F.Cu) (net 9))
 (segment (start 134.363 99.312) (end 136.395 99.312) (width 0.25) (layer F.Cu) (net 9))
 (segment (start 133.855 99.82) (end 134.363 99.312) (width 0.25) (layer F.Cu) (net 9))
 (segment (start 136.395 99.312) (end 136.903 99.82) (width 0.25) (layer F.Cu) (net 9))
 (segment (start 133.855 101.937) (end 133.855 99.82) (width 0.25) (layer F.Cu) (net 9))
 (segment (start 140.7585 101.452) (end 141.2665 100.944) (width 0.25) (layer F.Cu) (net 9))
 (segment (start 135.254 103.336) (end 133.855 101.937) (width 0.25) (layer F.Cu) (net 9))
 (segment (start 135.379 103.336) (end 135.254 103.336) (width 0.25) (layer F.Cu) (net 9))
 (segment (start 141.2665 100.944) (end 141.2665 97.3815) (width 0.25) (layer F.Cu) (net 9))
 (segment (start 136.903 99.82) (end 136.903 100.836) (width 0.25) (layer F.Cu) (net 9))
 (segment (start 136.903 100.836) (end 137.519 101.452) (width 0.25) (layer F.Cu) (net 9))
 (segment (start 141.2665 97.3815) (end 141.718932 96.929068) (width 0.25) (layer F.Cu) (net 9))
 (segment (start 137.519 101.452) (end 140.7585 101.452) (width 0.25) (layer F.Cu) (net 9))
 (segment (start 141.718932 96.929068) (end 156.40651 96.929068) (width 0.25) (layer F.Cu) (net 9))
 (segment (start 156.40651 96.929068) (end 157.16851 96.167068) (width 0.25) (layer F.Cu) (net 9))
 (segment (start 157.16851 96.167068) (end 157.16851 93.90751) (width 0.25) (layer F.Cu) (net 9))
 (segment (start 157.16851 93.90751) (end 156.95801 93.69701) (width 0.25) (layer F.Cu) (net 9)))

